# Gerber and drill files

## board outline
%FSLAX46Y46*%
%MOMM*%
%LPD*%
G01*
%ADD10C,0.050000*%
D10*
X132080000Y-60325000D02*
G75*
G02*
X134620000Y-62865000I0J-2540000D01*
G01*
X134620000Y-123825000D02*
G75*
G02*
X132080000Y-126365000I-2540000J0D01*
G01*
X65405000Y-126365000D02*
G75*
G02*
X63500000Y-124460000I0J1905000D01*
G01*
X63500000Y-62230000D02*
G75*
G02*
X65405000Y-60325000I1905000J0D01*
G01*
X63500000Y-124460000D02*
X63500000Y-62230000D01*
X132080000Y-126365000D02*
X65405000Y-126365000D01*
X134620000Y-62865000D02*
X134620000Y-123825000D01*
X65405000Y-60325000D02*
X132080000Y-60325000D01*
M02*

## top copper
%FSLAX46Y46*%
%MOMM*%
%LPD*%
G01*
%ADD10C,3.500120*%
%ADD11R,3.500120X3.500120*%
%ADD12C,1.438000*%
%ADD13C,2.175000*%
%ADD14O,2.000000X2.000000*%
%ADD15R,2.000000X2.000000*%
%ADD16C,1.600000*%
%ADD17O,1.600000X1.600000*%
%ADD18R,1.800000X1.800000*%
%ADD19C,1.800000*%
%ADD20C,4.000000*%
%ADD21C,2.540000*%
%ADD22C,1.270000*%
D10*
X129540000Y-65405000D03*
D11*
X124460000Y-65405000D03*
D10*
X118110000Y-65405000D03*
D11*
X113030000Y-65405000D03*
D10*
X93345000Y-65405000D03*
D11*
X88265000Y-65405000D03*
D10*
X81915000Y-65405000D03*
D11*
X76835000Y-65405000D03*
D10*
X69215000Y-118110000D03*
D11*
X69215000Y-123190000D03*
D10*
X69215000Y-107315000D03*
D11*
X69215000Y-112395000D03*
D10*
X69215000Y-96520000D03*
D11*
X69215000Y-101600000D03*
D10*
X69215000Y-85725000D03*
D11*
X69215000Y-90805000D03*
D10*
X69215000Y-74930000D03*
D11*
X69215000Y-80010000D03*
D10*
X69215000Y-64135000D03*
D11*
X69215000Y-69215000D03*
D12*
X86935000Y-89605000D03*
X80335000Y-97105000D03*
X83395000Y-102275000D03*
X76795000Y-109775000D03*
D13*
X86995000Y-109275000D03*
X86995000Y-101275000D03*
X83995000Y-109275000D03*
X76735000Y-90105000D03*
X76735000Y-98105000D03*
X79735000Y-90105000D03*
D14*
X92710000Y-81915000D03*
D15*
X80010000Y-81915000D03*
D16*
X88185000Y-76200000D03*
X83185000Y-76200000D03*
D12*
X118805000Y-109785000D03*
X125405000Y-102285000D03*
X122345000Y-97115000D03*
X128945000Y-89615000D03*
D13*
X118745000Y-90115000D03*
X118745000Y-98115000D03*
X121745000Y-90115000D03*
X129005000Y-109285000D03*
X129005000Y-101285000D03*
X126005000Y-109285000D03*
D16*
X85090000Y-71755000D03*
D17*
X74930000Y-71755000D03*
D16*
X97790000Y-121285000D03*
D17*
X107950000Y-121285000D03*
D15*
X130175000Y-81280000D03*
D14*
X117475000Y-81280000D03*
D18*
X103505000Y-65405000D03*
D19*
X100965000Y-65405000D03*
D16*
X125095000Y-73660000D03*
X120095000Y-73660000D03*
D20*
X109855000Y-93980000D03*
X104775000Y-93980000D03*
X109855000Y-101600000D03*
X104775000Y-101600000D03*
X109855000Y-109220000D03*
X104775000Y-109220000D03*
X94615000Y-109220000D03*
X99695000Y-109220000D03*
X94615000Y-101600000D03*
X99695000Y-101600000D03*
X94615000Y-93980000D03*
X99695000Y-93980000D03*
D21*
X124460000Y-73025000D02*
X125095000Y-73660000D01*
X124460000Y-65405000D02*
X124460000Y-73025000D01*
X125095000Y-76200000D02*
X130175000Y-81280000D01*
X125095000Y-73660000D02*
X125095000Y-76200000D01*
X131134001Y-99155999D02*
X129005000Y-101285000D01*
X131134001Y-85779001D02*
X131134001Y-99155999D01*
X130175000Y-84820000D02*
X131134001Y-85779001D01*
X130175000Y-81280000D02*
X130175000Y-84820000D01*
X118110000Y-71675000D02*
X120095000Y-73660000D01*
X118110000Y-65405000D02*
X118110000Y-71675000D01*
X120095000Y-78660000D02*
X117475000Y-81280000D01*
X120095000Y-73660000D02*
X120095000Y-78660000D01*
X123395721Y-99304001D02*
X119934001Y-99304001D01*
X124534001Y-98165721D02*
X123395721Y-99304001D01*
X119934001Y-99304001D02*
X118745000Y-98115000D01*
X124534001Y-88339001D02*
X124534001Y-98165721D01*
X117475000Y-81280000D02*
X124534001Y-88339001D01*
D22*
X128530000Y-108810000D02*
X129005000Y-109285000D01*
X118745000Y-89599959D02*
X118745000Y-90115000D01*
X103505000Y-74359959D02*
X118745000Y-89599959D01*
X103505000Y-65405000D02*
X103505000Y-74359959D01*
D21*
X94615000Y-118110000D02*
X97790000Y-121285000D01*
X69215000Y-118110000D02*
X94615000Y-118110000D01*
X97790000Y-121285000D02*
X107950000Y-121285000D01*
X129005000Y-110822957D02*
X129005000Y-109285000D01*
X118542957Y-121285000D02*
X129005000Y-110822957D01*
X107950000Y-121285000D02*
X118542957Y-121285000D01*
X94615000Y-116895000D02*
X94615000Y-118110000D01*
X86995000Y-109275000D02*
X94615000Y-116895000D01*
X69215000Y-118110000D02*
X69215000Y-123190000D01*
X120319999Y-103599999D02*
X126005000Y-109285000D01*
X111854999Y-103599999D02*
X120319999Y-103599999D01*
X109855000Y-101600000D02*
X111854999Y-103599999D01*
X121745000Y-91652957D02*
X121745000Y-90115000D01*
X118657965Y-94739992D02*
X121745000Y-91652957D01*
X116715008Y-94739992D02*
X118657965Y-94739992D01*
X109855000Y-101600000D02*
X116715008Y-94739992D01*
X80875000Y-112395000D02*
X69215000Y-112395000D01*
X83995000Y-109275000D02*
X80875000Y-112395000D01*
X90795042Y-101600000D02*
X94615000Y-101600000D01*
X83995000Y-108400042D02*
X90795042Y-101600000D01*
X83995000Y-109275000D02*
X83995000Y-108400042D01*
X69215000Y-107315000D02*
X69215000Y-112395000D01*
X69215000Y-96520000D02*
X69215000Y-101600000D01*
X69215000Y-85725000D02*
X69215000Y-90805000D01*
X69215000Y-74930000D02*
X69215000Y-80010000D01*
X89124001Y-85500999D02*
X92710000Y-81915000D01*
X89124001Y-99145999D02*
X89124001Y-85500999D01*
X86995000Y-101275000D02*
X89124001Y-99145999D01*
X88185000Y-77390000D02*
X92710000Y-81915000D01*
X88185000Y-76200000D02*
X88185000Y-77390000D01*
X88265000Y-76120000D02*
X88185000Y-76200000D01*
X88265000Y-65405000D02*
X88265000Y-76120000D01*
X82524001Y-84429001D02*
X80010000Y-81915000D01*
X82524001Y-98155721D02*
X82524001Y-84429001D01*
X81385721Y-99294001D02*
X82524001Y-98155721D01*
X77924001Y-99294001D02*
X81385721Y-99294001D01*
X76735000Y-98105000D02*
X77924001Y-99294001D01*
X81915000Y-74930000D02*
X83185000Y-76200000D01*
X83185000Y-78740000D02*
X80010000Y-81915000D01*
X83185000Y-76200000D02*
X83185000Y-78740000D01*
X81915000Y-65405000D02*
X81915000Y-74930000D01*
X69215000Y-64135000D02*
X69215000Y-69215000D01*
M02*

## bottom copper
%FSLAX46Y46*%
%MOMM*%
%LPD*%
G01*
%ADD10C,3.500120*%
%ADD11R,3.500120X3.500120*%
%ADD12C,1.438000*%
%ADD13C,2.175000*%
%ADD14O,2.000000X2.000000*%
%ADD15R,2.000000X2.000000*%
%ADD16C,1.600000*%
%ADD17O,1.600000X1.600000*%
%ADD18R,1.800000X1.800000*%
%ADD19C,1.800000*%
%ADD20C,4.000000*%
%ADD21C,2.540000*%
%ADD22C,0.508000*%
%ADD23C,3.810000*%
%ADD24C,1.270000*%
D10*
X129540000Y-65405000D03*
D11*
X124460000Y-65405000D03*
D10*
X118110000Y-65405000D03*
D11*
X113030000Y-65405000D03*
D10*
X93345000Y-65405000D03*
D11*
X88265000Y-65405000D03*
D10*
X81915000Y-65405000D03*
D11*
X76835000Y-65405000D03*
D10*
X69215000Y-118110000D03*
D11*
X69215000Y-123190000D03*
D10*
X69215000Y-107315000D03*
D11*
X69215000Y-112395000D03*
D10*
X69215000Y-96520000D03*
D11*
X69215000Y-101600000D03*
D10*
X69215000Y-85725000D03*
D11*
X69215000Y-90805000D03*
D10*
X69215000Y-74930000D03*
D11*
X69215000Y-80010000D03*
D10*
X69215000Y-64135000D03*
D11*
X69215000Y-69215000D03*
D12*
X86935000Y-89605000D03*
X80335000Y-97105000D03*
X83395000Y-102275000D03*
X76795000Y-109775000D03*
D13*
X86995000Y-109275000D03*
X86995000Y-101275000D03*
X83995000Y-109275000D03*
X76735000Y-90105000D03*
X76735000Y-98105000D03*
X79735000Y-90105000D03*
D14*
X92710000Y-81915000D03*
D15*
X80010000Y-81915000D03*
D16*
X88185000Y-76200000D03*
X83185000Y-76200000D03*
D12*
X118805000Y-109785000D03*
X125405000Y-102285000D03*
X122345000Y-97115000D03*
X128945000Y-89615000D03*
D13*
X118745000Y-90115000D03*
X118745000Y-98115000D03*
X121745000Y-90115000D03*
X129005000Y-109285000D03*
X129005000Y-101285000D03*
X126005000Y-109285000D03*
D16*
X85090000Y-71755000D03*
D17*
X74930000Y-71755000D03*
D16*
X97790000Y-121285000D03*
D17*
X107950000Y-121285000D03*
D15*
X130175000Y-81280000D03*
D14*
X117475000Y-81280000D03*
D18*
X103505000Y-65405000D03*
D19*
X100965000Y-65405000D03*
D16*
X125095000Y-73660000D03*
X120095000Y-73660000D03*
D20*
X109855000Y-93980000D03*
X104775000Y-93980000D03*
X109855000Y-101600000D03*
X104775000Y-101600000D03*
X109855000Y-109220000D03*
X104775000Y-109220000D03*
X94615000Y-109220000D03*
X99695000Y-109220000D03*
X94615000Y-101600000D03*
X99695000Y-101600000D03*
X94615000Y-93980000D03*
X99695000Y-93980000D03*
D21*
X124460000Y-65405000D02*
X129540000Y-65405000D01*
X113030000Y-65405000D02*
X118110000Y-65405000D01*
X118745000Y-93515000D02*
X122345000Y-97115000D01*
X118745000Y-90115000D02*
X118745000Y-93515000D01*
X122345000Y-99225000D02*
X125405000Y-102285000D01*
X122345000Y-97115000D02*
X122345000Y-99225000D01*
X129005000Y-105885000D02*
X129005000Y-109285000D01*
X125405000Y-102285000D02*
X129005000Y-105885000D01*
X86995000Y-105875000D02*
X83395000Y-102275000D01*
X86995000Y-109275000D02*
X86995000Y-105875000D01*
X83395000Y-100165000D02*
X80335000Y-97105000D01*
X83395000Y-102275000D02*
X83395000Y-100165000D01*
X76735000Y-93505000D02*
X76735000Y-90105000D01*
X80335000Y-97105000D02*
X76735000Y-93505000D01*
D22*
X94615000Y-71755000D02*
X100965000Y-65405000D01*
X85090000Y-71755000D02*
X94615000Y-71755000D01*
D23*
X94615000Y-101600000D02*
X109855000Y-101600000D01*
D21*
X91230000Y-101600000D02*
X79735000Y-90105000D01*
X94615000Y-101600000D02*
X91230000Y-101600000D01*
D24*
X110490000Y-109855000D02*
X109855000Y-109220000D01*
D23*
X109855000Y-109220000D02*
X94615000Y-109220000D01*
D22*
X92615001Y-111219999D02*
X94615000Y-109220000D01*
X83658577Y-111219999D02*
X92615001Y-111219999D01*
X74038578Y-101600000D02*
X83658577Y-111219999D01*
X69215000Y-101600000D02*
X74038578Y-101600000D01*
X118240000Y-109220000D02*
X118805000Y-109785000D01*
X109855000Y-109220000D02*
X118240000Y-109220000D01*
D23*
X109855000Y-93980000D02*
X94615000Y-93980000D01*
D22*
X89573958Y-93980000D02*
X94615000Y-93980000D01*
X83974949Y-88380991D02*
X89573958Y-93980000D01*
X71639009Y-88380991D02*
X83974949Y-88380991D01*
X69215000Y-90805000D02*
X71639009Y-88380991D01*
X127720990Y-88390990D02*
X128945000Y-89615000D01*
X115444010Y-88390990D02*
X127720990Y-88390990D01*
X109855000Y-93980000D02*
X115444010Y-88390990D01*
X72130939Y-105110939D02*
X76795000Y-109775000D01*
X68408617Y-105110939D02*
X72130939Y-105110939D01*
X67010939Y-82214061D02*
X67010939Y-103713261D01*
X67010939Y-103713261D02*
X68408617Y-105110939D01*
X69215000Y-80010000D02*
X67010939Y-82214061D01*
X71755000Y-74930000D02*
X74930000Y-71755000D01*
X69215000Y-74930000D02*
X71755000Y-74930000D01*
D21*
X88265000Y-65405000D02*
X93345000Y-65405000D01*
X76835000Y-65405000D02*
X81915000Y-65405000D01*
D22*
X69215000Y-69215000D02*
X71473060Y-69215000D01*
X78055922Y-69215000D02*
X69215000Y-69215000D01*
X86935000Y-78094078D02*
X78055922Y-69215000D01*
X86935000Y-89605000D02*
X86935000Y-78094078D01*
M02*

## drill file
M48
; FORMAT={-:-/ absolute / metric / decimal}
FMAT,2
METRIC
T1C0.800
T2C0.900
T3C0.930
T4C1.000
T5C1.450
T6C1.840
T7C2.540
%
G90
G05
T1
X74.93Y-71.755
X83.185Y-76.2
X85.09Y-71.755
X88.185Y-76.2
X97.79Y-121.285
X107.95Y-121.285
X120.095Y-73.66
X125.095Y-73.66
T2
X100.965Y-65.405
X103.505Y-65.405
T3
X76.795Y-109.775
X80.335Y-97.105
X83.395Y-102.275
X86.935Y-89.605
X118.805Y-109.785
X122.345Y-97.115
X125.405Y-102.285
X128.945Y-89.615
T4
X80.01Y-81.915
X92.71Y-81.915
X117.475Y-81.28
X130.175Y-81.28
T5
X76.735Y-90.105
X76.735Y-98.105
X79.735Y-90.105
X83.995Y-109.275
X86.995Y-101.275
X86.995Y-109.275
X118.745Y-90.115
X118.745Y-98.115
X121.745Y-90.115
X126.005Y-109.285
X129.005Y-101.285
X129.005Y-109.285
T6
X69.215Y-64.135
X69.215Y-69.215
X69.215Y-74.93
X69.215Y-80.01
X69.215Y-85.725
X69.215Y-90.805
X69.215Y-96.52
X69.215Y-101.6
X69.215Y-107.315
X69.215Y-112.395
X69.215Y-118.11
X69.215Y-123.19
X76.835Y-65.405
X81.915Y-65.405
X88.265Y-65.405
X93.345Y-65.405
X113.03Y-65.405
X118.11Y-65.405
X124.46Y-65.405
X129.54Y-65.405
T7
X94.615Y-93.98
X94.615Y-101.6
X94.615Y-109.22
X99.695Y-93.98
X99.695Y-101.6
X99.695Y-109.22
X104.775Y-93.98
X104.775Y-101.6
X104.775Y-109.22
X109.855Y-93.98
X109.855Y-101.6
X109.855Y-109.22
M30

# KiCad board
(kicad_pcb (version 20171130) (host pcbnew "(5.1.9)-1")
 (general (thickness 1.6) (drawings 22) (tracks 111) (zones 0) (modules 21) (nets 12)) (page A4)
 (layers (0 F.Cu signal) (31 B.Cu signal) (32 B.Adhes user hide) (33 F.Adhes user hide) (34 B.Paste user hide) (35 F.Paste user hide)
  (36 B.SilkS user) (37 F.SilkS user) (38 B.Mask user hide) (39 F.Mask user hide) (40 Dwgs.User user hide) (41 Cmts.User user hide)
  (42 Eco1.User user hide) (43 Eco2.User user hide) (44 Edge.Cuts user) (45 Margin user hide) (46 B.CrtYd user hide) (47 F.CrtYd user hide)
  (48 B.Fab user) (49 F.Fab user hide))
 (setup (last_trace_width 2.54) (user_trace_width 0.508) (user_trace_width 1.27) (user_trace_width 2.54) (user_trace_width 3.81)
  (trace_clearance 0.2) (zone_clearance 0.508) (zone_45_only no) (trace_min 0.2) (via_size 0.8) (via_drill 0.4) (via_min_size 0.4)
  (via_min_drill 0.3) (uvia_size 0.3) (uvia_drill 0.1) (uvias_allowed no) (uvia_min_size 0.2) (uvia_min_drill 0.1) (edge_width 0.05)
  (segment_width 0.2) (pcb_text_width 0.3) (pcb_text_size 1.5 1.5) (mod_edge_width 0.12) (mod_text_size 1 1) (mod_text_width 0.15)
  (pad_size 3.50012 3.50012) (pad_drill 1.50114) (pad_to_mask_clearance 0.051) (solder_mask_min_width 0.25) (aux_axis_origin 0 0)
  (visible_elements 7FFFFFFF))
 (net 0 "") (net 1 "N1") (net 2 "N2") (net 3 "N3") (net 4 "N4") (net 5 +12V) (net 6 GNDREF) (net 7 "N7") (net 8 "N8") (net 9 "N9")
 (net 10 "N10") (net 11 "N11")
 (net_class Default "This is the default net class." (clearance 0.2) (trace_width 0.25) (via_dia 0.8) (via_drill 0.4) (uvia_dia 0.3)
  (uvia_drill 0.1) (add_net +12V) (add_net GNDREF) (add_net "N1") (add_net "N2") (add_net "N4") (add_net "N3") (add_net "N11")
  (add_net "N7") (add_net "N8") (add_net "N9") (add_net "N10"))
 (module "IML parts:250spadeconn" (layer F.Cu) (at 124.46 65.405)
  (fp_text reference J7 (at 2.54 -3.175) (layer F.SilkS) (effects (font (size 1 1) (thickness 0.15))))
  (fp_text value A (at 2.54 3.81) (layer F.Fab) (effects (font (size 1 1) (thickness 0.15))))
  (pad 1 thru_hole circle (at 5.08 0) (size 3.50012 3.50012) (drill 1.84) (layers *.Cu *.Mask) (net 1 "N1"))
  (pad 1 thru_hole rect (at 0 0) (size 3.50012 3.50012) (drill 1.84) (layers *.Cu *.Mask) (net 1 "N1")))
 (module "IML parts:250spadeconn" (layer F.Cu) (at 113.03 65.405)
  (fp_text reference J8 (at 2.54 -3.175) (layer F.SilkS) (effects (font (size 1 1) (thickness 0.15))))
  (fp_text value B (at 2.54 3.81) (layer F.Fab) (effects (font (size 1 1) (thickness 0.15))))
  (pad 1 thru_hole circle (at 5.08 0) (size 3.50012 3.50012) (drill 1.84) (layers *.Cu *.Mask) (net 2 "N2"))
  (pad 1 thru_hole rect (at 0 0) (size 3.50012 3.50012) (drill 1.84) (layers *.Cu *.Mask) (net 2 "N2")))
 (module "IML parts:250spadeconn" (layer F.Cu) (at 88.265 65.405)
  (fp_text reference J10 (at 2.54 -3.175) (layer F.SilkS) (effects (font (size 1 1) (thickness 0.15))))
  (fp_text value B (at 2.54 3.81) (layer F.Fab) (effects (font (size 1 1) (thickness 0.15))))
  (pad 1 thru_hole circle (at 5.08 0) (size 3.50012 3.50012) (drill 1.84) (layers *.Cu *.Mask) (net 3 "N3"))
  (pad 1 thru_hole rect (at 0 0) (size 3.50012 3.50012) (drill 1.84) (layers *.Cu *.Mask) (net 3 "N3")))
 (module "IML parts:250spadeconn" (layer F.Cu) (at 76.835 65.405)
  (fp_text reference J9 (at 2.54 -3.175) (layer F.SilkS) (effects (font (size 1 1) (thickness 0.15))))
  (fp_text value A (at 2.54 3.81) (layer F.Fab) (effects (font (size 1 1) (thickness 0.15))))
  (pad 1 thru_hole circle (at 5.08 0) (size 3.50012 3.50012) (drill 1.84) (layers *.Cu *.Mask) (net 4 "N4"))
  (pad 1 thru_hole rect (at 0 0) (size 3.50012 3.50012) (drill 1.84) (layers *.Cu *.Mask) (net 4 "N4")))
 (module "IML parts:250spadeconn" (layer F.Cu) (at 69.215 123.19 90)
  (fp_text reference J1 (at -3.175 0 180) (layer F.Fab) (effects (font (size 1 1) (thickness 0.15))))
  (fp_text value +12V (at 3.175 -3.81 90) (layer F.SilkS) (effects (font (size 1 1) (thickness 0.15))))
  (pad 1 thru_hole circle (at 5.08 0 90) (size 3.50012 3.50012) (drill 1.84) (layers *.Cu *.Mask) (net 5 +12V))
  (pad 1 thru_hole rect (at 0 0 90) (size 3.50012 3.50012) (drill 1.84) (layers *.Cu *.Mask) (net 5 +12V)))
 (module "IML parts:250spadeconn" (layer F.Cu) (at 69.215 112.395 90)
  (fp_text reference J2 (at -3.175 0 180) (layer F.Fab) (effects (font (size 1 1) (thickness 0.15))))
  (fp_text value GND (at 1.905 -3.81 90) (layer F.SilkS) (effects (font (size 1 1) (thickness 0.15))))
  (pad 1 thru_hole circle (at 5.08 0 90) (size 3.50012 3.50012) (drill 1.84) (layers *.Cu *.Mask) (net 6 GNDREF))
  (pad 1 thru_hole rect (at 0 0 90) (size 3.50012 3.50012) (drill 1.84) (layers *.Cu *.Mask) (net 6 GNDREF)))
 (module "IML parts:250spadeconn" (layer F.Cu) (at 69.215 101.6 90)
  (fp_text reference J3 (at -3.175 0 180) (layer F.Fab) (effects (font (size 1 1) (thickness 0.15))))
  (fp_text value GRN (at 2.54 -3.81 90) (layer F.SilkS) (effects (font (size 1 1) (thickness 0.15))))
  (pad 1 thru_hole circle (at 5.08 0 90) (size 3.50012 3.50012) (drill 1.84) (layers *.Cu *.Mask) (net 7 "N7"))
  (pad 1 thru_hole rect (at 0 0 90) (size 3.50012 3.50012) (drill 1.84) (layers *.Cu *.Mask) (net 7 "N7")))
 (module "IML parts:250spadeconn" (layer F.Cu) (at 69.215 90.805 90)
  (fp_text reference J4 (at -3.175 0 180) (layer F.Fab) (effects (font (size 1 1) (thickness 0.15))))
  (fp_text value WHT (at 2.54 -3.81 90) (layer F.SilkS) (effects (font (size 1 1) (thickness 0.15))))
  (pad 1 thru_hole circle (at 5.08 0 90) (size 3.50012 3.50012) (drill 1.84) (layers *.Cu *.Mask) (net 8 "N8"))
  (pad 1 thru_hole rect (at 0 0 90) (size 3.50012 3.50012) (drill 1.84) (layers *.Cu *.Mask) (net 8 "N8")))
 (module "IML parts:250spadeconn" (layer F.Cu) (at 69.215 80.01 90)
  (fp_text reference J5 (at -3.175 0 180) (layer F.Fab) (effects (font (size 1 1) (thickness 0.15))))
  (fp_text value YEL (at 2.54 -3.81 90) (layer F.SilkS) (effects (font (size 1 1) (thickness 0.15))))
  (pad 1 thru_hole circle (at 5.08 0 90) (size 3.50012 3.50012) (drill 1.84) (layers *.Cu *.Mask) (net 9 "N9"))
  (pad 1 thru_hole rect (at 0 0 90) (size 3.50012 3.50012) (drill 1.84) (layers *.Cu *.Mask) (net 9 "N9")))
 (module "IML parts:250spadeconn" (layer F.Cu) (at 69.215 69.215 90)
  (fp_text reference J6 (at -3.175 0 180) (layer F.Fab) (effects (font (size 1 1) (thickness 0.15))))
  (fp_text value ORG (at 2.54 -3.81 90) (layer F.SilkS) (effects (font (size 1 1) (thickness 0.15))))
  (pad 1 thru_hole circle (at 5.08 0 90) (size 3.50012 3.50012) (drill 1.84) (layers *.Cu *.Mask) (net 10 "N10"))
  (pad 1 thru_hole rect (at 0 0 90) (size 3.50012 3.50012) (drill 1.84) (layers *.Cu *.Mask) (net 10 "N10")))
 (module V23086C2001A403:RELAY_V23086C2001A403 (layer F.Cu) (at 81.915 99.695 270)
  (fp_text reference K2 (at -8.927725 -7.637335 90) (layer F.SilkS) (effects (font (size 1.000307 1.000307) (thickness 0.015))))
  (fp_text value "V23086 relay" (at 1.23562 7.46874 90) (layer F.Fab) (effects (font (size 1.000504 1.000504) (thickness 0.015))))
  (pad 22 thru_hole circle (at -10.09 -5.02 270) (size 1.438 1.438) (drill 0.93) (layers *.Cu *.Mask) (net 10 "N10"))
  (pad 21 thru_hole circle (at -2.59 1.58 270) (size 1.438 1.438) (drill 0.93) (layers *.Cu *.Mask) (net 5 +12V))
  (pad 11 thru_hole circle (at 2.58 -1.48 270) (size 1.438 1.438) (drill 0.93) (layers *.Cu *.Mask) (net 5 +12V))
  (pad 12 thru_hole circle (at 10.08 5.12 270) (size 1.438 1.438) (drill 0.93) (layers *.Cu *.Mask) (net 9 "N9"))
  (pad 13 thru_hole circle (at 9.58 -5.08 270) (size 2.175 2.175) (drill 1.45) (layers *.Cu *.Mask) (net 5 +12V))
  (pad 14 thru_hole circle (at 1.58 -5.08 270) (size 2.175 2.175) (drill 1.45) (layers *.Cu *.Mask) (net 3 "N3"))
  (pad 15 thru_hole circle (at 9.58 -2.08 270) (size 2.175 2.175) (drill 1.45) (layers *.Cu *.Mask) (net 6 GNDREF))
  (pad 23 thru_hole circle (at -9.59 5.18 270) (size 2.175 2.175) (drill 1.45) (layers *.Cu *.Mask) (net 5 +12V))
  (pad 24 thru_hole circle (at -1.59 5.18 270) (size 2.175 2.175) (drill 1.45) (layers *.Cu *.Mask) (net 4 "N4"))
  (pad 25 thru_hole circle (at -9.59 2.18 270) (size 2.175 2.175) (drill 1.45) (layers *.Cu *.Mask) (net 6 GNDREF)))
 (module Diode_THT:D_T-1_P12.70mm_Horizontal (layer F.Cu) (at 80.01 81.915)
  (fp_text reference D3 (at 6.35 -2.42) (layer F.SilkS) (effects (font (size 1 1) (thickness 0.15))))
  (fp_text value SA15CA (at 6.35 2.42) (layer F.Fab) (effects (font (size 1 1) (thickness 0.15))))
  (pad 2 thru_hole oval (at 12.7 0) (size 2 2) (drill 1) (layers *.Cu *.Mask) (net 3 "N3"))
  (pad 1 thru_hole rect (at 0 0) (size 2 2) (drill 1) (layers *.Cu *.Mask) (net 4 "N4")))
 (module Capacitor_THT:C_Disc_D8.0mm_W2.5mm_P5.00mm (layer F.Cu) (at 83.185 76.2)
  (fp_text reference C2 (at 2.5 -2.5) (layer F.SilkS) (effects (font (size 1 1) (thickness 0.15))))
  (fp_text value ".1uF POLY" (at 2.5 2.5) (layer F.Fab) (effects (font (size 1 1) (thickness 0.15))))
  (pad 2 thru_hole circle (at 5 0) (size 1.6 1.6) (drill 0.8) (layers *.Cu *.Mask) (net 3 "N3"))
  (pad 1 thru_hole circle (at 0 0) (size 1.6 1.6) (drill 0.8) (layers *.Cu *.Mask) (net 4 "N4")))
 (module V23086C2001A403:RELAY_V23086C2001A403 (layer F.Cu) (at 123.825 99.695 90)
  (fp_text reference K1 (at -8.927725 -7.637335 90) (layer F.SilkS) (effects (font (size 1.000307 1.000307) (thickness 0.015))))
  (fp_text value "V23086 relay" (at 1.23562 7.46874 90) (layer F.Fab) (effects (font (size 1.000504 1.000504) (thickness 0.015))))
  (pad 22 thru_hole circle (at -10.09 -5.02 90) (size 1.438 1.438) (drill 0.93) (layers *.Cu *.Mask) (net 7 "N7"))
  (pad 21 thru_hole circle (at -2.59 1.58 90) (size 1.438 1.438) (drill 0.93) (layers *.Cu *.Mask) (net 5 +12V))
  (pad 11 thru_hole circle (at 2.58 -1.48 90) (size 1.438 1.438) (drill 0.93) (layers *.Cu *.Mask) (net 5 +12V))
  (pad 12 thru_hole circle (at 10.08 5.12 90) (size 1.438 1.438) (drill 0.93) (layers *.Cu *.Mask) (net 8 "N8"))
  (pad 13 thru_hole circle (at 9.58 -5.08 90) (size 2.175 2.175) (drill 1.45) (layers *.Cu *.Mask) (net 5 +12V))
  (pad 14 thru_hole circle (at 1.58 -5.08 90) (size 2.175 2.175) (drill 1.45) (layers *.Cu *.Mask) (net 2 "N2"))
  (pad 15 thru_hole circle (at 9.58 -2.08 90) (size 2.175 2.175) (drill 1.45) (layers *.Cu *.Mask) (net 6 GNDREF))
  (pad 23 thru_hole circle (at -9.59 5.18 90) (size 2.175 2.175) (drill 1.45) (layers *.Cu *.Mask) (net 5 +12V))
  (pad 24 thru_hole circle (at -1.59 5.18 90) (size 2.175 2.175) (drill 1.45) (layers *.Cu *.Mask) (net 1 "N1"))
  (pad 25 thru_hole circle (at -9.59 2.18 90) (size 2.175 2.175) (drill 1.45) (layers *.Cu *.Mask) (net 6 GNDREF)))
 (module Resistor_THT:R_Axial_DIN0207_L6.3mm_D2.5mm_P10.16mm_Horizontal (layer F.Cu) (at 85.09 71.755 180)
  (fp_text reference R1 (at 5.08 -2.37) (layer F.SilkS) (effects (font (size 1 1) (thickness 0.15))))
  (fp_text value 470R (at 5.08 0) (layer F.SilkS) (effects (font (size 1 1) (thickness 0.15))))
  (pad 1 thru_hole circle (at 0 0 180) (size 1.6 1.6) (drill 0.8) (layers *.Cu *.Mask) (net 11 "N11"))
  (pad 2 thru_hole oval (at 10.16 0 180) (size 1.6 1.6) (drill 0.8) (layers *.Cu *.Mask) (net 9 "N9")))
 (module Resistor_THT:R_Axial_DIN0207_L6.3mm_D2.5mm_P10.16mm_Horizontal (layer F.Cu) (at 97.79 121.285)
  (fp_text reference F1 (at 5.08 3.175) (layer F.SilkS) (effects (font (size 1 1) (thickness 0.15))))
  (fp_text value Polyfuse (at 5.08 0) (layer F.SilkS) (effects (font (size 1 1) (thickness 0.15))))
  (pad 1 thru_hole circle (at 0 0) (size 1.6 1.6) (drill 0.8) (layers *.Cu *.Mask) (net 5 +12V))
  (pad 2 thru_hole oval (at 10.16 0) (size 1.6 1.6) (drill 0.8) (layers *.Cu *.Mask) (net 5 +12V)))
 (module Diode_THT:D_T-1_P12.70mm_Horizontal (layer F.Cu) (at 130.175 81.28 180)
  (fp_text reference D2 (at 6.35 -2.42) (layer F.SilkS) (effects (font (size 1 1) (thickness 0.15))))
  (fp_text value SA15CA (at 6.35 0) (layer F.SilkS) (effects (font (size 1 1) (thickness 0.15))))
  (pad 1 thru_hole rect (at 0 0 180) (size 2 2) (drill 1) (layers *.Cu *.Mask) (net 1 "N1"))
  (pad 2 thru_hole oval (at 12.7 0 180) (size 2 2) (drill 1) (layers *.Cu *.Mask) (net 2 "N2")))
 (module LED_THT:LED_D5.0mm (layer F.Cu) (at 103.505 65.405 180)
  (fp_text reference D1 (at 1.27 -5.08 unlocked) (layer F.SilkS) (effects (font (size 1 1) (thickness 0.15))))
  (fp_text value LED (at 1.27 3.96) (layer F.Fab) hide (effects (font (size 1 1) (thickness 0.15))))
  (pad 1 thru_hole rect (at 0 0 180) (size 1.8 1.8) (drill 0.9) (layers *.Cu *.Mask) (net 5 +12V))
  (pad 2 thru_hole circle (at 2.54 0 180) (size 1.8 1.8) (drill 0.9) (layers *.Cu *.Mask) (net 11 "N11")))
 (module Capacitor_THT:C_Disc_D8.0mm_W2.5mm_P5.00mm (layer F.Cu) (at 125.095 73.66 180)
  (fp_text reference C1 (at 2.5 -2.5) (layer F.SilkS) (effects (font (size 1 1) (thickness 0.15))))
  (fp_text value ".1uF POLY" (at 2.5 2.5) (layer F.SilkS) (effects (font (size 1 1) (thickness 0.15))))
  (pad 1 thru_hole circle (at 0 0 180) (size 1.6 1.6) (drill 0.8) (layers *.Cu *.Mask) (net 1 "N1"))
  (pad 2 thru_hole circle (at 5 0 180) (size 1.6 1.6) (drill 0.8) (layers *.Cu *.Mask) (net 2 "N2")))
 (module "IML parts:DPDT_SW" (layer F.Cu) (at 107.315 101.6 90)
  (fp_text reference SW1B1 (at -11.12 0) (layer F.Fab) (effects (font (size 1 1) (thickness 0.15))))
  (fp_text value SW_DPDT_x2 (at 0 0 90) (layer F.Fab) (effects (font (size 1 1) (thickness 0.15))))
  (pad 3 thru_hole circle (at 7.62 2.54 90) (size 4 4) (drill 2.54) (layers *.Cu *.Mask) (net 8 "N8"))
  (pad 3 thru_hole circle (at 7.62 -2.54 90) (size 4 4) (drill 2.54) (layers *.Cu *.Mask) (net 8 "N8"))
  (pad 2 thru_hole circle (at 0 2.54 90) (size 4 4) (drill 2.54) (layers *.Cu *.Mask) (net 6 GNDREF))
  (pad 2 thru_hole circle (at 0 -2.54 90) (size 4 4) (drill 2.54) (layers *.Cu *.Mask) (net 6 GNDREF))
  (pad 1 thru_hole circle (at -7.62 2.54 90) (size 4 4) (drill 2.54) (layers *.Cu *.Mask) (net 7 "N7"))
  (pad 1 thru_hole circle (at -7.62 -2.54 90) (size 4 4) (drill 2.54) (layers *.Cu *.Mask) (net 7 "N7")))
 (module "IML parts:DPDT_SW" (layer F.Cu) (at 97.155 101.6 90)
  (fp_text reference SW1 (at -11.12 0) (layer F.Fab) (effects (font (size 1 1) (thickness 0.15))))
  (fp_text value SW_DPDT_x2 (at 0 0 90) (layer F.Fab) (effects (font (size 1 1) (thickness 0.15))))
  (pad 1 thru_hole circle (at -7.62 -2.54 90) (size 4 4) (drill 2.54) (layers *.Cu *.Mask) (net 7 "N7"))
  (pad 1 thru_hole circle (at -7.62 2.54 90) (size 4 4) (drill 2.54) (layers *.Cu *.Mask) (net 7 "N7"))
  (pad 2 thru_hole circle (at 0 -2.54 90) (size 4 4) (drill 2.54) (layers *.Cu *.Mask) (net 6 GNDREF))
  (pad 2 thru_hole circle (at 0 2.54 90) (size 4 4) (drill 2.54) (layers *.Cu *.Mask) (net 6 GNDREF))
  (pad 3 thru_hole circle (at 7.62 -2.54 90) (size 4 4) (drill 2.54) (layers *.Cu *.Mask) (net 8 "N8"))
  (pad 3 thru_hole circle (at 7.62 2.54 90) (size 4 4) (drill 2.54) (layers *.Cu *.Mask) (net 8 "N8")))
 (gr_arc (start 132.08 62.865) (end 134.62 62.865) (angle -90) (layer Edge.Cuts) (width 0.05))
 (gr_arc (start 132.08 123.825) (end 132.08 126.365) (angle -90) (layer Edge.Cuts) (width 0.05))
 (gr_arc (start 65.405 124.46) (end 63.5 124.46) (angle -90) (layer Edge.Cuts) (width 0.05))
 (gr_arc (start 65.405 62.23) (end 65.405 60.325) (angle -90) (layer Edge.Cuts) (width 0.05))
 (gr_line (start 63.5 124.46) (end 63.5 62.23) (layer Edge.Cuts) (width 0.05))
 (gr_line (start 132.08 126.365) (end 65.405 126.365) (layer Edge.Cuts) (width 0.05))
 (gr_line (start 134.62 62.865) (end 134.62 123.825) (layer Edge.Cuts) (width 0.05))
 (gr_line (start 65.405 60.325) (end 132.08 60.325) (layer Edge.Cuts) (width 0.05))
 (segment (start 124.46 73.025) (end 125.095 73.66) (width 2.54) (layer F.Cu) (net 1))
 (segment (start 124.46 65.405) (end 124.46 73.025) (width 2.54) (layer F.Cu) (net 1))
 (segment (start 125.095 76.2) (end 130.175 81.28) (width 2.54) (layer F.Cu) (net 1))
 (segment (start 125.095 73.66) (end 125.095 76.2) (width 2.54) (layer F.Cu) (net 1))
 (segment (start 131.134001 99.155999) (end 129.005 101.285) (width 2.54) (layer F.Cu) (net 1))
 (segment (start 131.134001 85.779001) (end 131.134001 99.155999) (width 2.54) (layer F.Cu) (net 1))
 (segment (start 130.175 84.82) (end 131.134001 85.779001) (width 2.54) (layer F.Cu) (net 1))
 (segment (start 130.175 81.28) (end 130.175 84.82) (width 2.54) (layer F.Cu) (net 1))
 (segment (start 124.46 65.405) (end 129.54 65.405) (width 2.54) (layer B.Cu) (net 1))
 (segment (start 118.11 71.675) (end 120.095 73.66) (width 2.54) (layer F.Cu) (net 2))
 (segment (start 118.11 65.405) (end 118.11 71.675) (width 2.54) (layer F.Cu) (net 2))
 (segment (start 120.095 78.66) (end 117.475 81.28) (width 2.54) (layer F.Cu) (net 2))
 (segment (start 120.095 73.66) (end 120.095 78.66) (width 2.54) (layer F.Cu) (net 2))
 (segment (start 123.395721 99.304001) (end 119.934001 99.304001) (width 2.54) (layer F.Cu) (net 2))
 (segment (start 124.534001 98.165721) (end 123.395721 99.304001) (width 2.54) (layer F.Cu) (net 2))
 (segment (start 119.934001 99.304001) (end 118.745 98.115) (width 2.54) (layer F.Cu) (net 2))
 (segment (start 124.534001 88.339001) (end 124.534001 98.165721) (width 2.54) (layer F.Cu) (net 2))
 (segment (start 117.475 81.28) (end 124.534001 88.339001) (width 2.54) (layer F.Cu) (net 2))
 (segment (start 113.03 65.405) (end 118.11 65.405) (width 2.54) (layer B.Cu) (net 2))
 (segment (start 128.53 108.81) (end 129.005 109.285) (width 1.27) (layer F.Cu) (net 5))
 (segment (start 118.745 93.515) (end 122.345 97.115) (width 2.54) (layer B.Cu) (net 5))
 (segment (start 118.745 90.115) (end 118.745 93.515) (width 2.54) (layer B.Cu) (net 5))
 (segment (start 122.345 99.225) (end 125.405 102.285) (width 2.54) (layer B.Cu) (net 5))
 (segment (start 122.345 97.115) (end 122.345 99.225) (width 2.54) (layer B.Cu) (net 5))
 (segment (start 129.005 105.885) (end 129.005 109.285) (width 2.54) (layer B.Cu) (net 5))
 (segment (start 125.405 102.285) (end 129.005 105.885) (width 2.54) (layer B.Cu) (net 5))
 (segment (start 118.745 89.599959) (end 118.745 90.115) (width 1.27) (layer F.Cu) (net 5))
 (segment (start 103.505 74.359959) (end 118.745 89.599959) (width 1.27) (layer F.Cu) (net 5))
 (segment (start 103.505 65.405) (end 103.505 74.359959) (width 1.27) (layer F.Cu) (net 5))
 (segment (start 86.995 105.875) (end 83.395 102.275) (width 2.54) (layer B.Cu) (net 5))
 (segment (start 86.995 109.275) (end 86.995 105.875) (width 2.54) (layer B.Cu) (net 5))
 (segment (start 83.395 100.165) (end 80.335 97.105) (width 2.54) (layer B.Cu) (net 5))
 (segment (start 83.395 102.275) (end 83.395 100.165) (width 2.54) (layer B.Cu) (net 5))
 (segment (start 76.735 93.505) (end 76.735 90.105) (width 2.54) (layer B.Cu) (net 5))
 (segment (start 80.335 97.105) (end 76.735 93.505) (width 2.54) (layer B.Cu) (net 5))
 (segment (start 94.615 118.11) (end 97.79 121.285) (width 2.54) (layer F.Cu) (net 5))
 (segment (start 69.215 118.11) (end 94.615 118.11) (width 2.54) (layer F.Cu) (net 5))
 (segment (start 97.79 121.285) (end 107.95 121.285) (width 2.54) (layer F.Cu) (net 5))
 (segment (start 129.005 110.822957) (end 129.005 109.285) (width 2.54) (layer F.Cu) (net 5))
 (segment (start 118.542957 121.285) (end 129.005 110.822957) (width 2.54) (layer F.Cu) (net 5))
 (segment (start 107.95 121.285) (end 118.542957 121.285) (width 2.54) (layer F.Cu) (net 5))
 (segment (start 94.615 116.895) (end 94.615 118.11) (width 2.54) (layer F.Cu) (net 5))
 (segment (start 86.995 109.275) (end 94.615 116.895) (width 2.54) (layer F.Cu) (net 5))
 (segment (start 69.215 118.11) (end 69.215 123.19) (width 2.54) (layer F.Cu) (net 5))
 (segment (start 94.615 71.755) (end 100.965 65.405) (width 0.508) (layer B.Cu) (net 11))
 (segment (start 85.09 71.755) (end 94.615 71.755) (width 0.508) (layer B.Cu) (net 11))
 (segment (start 94.615 101.6) (end 109.855 101.6) (width 3.81) (layer B.Cu) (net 6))
 (segment (start 120.319999 103.599999) (end 126.005 109.285) (width 2.54) (layer F.Cu) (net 6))
 (segment (start 111.854999 103.599999) (end 120.319999 103.599999) (width 2.54) (layer F.Cu) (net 6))
 (segment (start 109.855 101.6) (end 111.854999 103.599999) (width 2.54) (layer F.Cu) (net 6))
 (segment (start 121.745 91.652957) (end 121.745 90.115) (width 2.54) (layer F.Cu) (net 6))
 (segment (start 118.657965 94.739992) (end 121.745 91.652957) (width 2.54) (layer F.Cu) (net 6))
 (segment (start 116.715008 94.739992) (end 118.657965 94.739992) (width 2.54) (layer F.Cu) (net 6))
 (segment (start 109.855 101.6) (end 116.715008 94.739992) (width 2.54) (layer F.Cu) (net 6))
 (segment (start 80.875 112.395) (end 69.215 112.395) (width 2.54) (layer F.Cu) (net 6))
 (segment (start 83.995 109.275) (end 80.875 112.395) (width 2.54) (layer F.Cu) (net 6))
 (segment (start 91.23 101.6) (end 79.735 90.105) (width 2.54) (layer B.Cu) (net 6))
 (segment (start 94.615 101.6) (end 91.23 101.6) (width 2.54) (layer B.Cu) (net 6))
 (segment (start 90.795042 101.6) (end 94.615 101.6) (width 2.54) (layer F.Cu) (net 6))
 (segment (start 83.995 108.400042) (end 90.795042 101.6) (width 2.54) (layer F.Cu) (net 6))
 (segment (start 83.995 109.275) (end 83.995 108.400042) (width 2.54) (layer F.Cu) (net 6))
 (segment (start 69.215 107.315) (end 69.215 112.395) (width 2.54) (layer F.Cu) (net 6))
 (segment (start 110.49 109.855) (end 109.855 109.22) (width 1.27) (layer B.Cu) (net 7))
 (segment (start 109.855 109.22) (end 94.615 109.22) (width 3.81) (layer B.Cu) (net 7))
 (segment (start 92.615001 111.219999) (end 94.615 109.22) (width 0.508) (layer B.Cu) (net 7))
 (segment (start 83.658577 111.219999) (end 92.615001 111.219999) (width 0.508) (layer B.Cu) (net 7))
 (segment (start 74.038578 101.6) (end 83.658577 111.219999) (width 0.508) (layer B.Cu) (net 7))
 (segment (start 69.215 101.6) (end 74.038578 101.6) (width 0.508) (layer B.Cu) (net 7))
 (segment (start 118.24 109.22) (end 118.805 109.785) (width 0.508) (layer B.Cu) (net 7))
 (segment (start 109.855 109.22) (end 118.24 109.22) (width 0.508) (layer B.Cu) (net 7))
 (segment (start 69.215 96.52) (end 69.215 101.6) (width 2.54) (layer F.Cu) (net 7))
 (segment (start 109.855 93.98) (end 94.615 93.98) (width 3.81) (layer B.Cu) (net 8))
 (segment (start 89.573958 93.98) (end 94.615 93.98) (width 0.508) (layer B.Cu) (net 8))
 (segment (start 83.974949 88.380991) (end 89.573958 93.98) (width 0.508) (layer B.Cu) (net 8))
 (segment (start 71.639009 88.380991) (end 83.974949 88.380991) (width 0.508) (layer B.Cu) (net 8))
 (segment (start 69.215 90.805) (end 71.639009 88.380991) (width 0.508) (layer B.Cu) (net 8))
 (segment (start 127.72099 88.39099) (end 128.945 89.615) (width 0.508) (layer B.Cu) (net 8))
 (segment (start 115.44401 88.39099) (end 127.72099 88.39099) (width 0.508) (layer B.Cu) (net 8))
 (segment (start 109.855 93.98) (end 115.44401 88.39099) (width 0.508) (layer B.Cu) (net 8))
 (segment (start 69.215 85.725) (end 69.215 90.805) (width 2.54) (layer F.Cu) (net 8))
 (segment (start 72.130939 105.110939) (end 76.795 109.775) (width 0.508) (layer B.Cu) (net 9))
 (segment (start 68.408617 105.110939) (end 72.130939 105.110939) (width 0.508) (layer B.Cu) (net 9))
 (segment (start 67.010939 82.214061) (end 67.010939 103.713261) (width 0.508) (layer B.Cu) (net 9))
 (segment (start 67.010939 103.713261) (end 68.408617 105.110939) (width 0.508) (layer B.Cu) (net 9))
 (segment (start 69.215 80.01) (end 67.010939 82.214061) (width 0.508) (layer B.Cu) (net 9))
 (segment (start 71.755 74.93) (end 74.93 71.755) (width 0.508) (layer B.Cu) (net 9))
 (segment (start 69.215 74.93) (end 71.755 74.93) (width 0.508) (layer B.Cu) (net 9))
 (segment (start 69.215 74.93) (end 69.215 80.01) (width 2.54) (layer F.Cu) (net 9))
 (segment (start 89.124001 85.500999) (end 92.71 81.915) (width 2.54) (layer F.Cu) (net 3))
 (segment (start 89.124001 99.145999) (end 89.124001 85.500999) (width 2.54) (layer F.Cu) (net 3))
 (segment (start 86.995 101.275) (end 89.124001 99.145999) (width 2.54) (layer F.Cu) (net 3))
 (segment (start 88.185 77.39) (end 92.71 81.915) (width 2.54) (layer F.Cu) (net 3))
 (segment (start 88.185 76.2) (end 88.185 77.39) (width 2.54) (layer F.Cu) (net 3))
 (segment (start 88.265 76.12) (end 88.185 76.2) (width 2.54) (layer F.Cu) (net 3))
 (segment (start 88.265 65.405) (end 88.265 76.12) (width 2.54) (layer F.Cu) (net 3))
 (segment (start 88.265 65.405) (end 93.345 65.405) (width 2.54) (layer B.Cu) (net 3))
 (segment (start 82.524001 84.429001) (end 80.01 81.915) (width 2.54) (layer F.Cu) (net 4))
 (segment (start 82.524001 98.155721) (end 82.524001 84.429001) (width 2.54) (layer F.Cu) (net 4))
 (segment (start 81.385721 99.294001) (end 82.524001 98.155721) (width 2.54) (layer F.Cu) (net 4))
 (segment (start 77.924001 99.294001) (end 81.385721 99.294001) (width 2.54) (layer F.Cu) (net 4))
 (segment (start 76.735 98.105) (end 77.924001 99.294001) (width 2.54) (layer F.Cu) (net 4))
 (segment (start 81.915 74.93) (end 83.185 76.2) (width 2.54) (layer F.Cu) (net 4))
 (segment (start 83.185 78.74) (end 80.01 81.915) (width 2.54) (layer F.Cu) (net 4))
 (segment (start 83.185 76.2) (end 83.185 78.74) (width 2.54) (layer F.Cu) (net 4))
 (segment (start 81.915 65.405) (end 81.915 74.93) (width 2.54) (layer F.Cu) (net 4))
 (segment (start 76.835 65.405) (end 81.915 65.405) (width 2.54) (layer B.Cu) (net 4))
 (segment (start 69.215 69.215) (end 71.47306 69.215) (width 0.508) (layer B.Cu) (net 10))
 (segment (start 78.055922 69.215) (end 69.215 69.215) (width 0.508) (layer B.Cu) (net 10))
 (segment (start 86.935 78.094078) (end 78.055922 69.215) (width 0.508) (layer B.Cu) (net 10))
 (segment (start 86.935 89.605) (end 86.935 78.094078) (width 0.508) (layer B.Cu) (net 10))
 (segment (start 69.215 64.135) (end 69.215 69.215) (width 2.54) (layer F.Cu) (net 10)))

